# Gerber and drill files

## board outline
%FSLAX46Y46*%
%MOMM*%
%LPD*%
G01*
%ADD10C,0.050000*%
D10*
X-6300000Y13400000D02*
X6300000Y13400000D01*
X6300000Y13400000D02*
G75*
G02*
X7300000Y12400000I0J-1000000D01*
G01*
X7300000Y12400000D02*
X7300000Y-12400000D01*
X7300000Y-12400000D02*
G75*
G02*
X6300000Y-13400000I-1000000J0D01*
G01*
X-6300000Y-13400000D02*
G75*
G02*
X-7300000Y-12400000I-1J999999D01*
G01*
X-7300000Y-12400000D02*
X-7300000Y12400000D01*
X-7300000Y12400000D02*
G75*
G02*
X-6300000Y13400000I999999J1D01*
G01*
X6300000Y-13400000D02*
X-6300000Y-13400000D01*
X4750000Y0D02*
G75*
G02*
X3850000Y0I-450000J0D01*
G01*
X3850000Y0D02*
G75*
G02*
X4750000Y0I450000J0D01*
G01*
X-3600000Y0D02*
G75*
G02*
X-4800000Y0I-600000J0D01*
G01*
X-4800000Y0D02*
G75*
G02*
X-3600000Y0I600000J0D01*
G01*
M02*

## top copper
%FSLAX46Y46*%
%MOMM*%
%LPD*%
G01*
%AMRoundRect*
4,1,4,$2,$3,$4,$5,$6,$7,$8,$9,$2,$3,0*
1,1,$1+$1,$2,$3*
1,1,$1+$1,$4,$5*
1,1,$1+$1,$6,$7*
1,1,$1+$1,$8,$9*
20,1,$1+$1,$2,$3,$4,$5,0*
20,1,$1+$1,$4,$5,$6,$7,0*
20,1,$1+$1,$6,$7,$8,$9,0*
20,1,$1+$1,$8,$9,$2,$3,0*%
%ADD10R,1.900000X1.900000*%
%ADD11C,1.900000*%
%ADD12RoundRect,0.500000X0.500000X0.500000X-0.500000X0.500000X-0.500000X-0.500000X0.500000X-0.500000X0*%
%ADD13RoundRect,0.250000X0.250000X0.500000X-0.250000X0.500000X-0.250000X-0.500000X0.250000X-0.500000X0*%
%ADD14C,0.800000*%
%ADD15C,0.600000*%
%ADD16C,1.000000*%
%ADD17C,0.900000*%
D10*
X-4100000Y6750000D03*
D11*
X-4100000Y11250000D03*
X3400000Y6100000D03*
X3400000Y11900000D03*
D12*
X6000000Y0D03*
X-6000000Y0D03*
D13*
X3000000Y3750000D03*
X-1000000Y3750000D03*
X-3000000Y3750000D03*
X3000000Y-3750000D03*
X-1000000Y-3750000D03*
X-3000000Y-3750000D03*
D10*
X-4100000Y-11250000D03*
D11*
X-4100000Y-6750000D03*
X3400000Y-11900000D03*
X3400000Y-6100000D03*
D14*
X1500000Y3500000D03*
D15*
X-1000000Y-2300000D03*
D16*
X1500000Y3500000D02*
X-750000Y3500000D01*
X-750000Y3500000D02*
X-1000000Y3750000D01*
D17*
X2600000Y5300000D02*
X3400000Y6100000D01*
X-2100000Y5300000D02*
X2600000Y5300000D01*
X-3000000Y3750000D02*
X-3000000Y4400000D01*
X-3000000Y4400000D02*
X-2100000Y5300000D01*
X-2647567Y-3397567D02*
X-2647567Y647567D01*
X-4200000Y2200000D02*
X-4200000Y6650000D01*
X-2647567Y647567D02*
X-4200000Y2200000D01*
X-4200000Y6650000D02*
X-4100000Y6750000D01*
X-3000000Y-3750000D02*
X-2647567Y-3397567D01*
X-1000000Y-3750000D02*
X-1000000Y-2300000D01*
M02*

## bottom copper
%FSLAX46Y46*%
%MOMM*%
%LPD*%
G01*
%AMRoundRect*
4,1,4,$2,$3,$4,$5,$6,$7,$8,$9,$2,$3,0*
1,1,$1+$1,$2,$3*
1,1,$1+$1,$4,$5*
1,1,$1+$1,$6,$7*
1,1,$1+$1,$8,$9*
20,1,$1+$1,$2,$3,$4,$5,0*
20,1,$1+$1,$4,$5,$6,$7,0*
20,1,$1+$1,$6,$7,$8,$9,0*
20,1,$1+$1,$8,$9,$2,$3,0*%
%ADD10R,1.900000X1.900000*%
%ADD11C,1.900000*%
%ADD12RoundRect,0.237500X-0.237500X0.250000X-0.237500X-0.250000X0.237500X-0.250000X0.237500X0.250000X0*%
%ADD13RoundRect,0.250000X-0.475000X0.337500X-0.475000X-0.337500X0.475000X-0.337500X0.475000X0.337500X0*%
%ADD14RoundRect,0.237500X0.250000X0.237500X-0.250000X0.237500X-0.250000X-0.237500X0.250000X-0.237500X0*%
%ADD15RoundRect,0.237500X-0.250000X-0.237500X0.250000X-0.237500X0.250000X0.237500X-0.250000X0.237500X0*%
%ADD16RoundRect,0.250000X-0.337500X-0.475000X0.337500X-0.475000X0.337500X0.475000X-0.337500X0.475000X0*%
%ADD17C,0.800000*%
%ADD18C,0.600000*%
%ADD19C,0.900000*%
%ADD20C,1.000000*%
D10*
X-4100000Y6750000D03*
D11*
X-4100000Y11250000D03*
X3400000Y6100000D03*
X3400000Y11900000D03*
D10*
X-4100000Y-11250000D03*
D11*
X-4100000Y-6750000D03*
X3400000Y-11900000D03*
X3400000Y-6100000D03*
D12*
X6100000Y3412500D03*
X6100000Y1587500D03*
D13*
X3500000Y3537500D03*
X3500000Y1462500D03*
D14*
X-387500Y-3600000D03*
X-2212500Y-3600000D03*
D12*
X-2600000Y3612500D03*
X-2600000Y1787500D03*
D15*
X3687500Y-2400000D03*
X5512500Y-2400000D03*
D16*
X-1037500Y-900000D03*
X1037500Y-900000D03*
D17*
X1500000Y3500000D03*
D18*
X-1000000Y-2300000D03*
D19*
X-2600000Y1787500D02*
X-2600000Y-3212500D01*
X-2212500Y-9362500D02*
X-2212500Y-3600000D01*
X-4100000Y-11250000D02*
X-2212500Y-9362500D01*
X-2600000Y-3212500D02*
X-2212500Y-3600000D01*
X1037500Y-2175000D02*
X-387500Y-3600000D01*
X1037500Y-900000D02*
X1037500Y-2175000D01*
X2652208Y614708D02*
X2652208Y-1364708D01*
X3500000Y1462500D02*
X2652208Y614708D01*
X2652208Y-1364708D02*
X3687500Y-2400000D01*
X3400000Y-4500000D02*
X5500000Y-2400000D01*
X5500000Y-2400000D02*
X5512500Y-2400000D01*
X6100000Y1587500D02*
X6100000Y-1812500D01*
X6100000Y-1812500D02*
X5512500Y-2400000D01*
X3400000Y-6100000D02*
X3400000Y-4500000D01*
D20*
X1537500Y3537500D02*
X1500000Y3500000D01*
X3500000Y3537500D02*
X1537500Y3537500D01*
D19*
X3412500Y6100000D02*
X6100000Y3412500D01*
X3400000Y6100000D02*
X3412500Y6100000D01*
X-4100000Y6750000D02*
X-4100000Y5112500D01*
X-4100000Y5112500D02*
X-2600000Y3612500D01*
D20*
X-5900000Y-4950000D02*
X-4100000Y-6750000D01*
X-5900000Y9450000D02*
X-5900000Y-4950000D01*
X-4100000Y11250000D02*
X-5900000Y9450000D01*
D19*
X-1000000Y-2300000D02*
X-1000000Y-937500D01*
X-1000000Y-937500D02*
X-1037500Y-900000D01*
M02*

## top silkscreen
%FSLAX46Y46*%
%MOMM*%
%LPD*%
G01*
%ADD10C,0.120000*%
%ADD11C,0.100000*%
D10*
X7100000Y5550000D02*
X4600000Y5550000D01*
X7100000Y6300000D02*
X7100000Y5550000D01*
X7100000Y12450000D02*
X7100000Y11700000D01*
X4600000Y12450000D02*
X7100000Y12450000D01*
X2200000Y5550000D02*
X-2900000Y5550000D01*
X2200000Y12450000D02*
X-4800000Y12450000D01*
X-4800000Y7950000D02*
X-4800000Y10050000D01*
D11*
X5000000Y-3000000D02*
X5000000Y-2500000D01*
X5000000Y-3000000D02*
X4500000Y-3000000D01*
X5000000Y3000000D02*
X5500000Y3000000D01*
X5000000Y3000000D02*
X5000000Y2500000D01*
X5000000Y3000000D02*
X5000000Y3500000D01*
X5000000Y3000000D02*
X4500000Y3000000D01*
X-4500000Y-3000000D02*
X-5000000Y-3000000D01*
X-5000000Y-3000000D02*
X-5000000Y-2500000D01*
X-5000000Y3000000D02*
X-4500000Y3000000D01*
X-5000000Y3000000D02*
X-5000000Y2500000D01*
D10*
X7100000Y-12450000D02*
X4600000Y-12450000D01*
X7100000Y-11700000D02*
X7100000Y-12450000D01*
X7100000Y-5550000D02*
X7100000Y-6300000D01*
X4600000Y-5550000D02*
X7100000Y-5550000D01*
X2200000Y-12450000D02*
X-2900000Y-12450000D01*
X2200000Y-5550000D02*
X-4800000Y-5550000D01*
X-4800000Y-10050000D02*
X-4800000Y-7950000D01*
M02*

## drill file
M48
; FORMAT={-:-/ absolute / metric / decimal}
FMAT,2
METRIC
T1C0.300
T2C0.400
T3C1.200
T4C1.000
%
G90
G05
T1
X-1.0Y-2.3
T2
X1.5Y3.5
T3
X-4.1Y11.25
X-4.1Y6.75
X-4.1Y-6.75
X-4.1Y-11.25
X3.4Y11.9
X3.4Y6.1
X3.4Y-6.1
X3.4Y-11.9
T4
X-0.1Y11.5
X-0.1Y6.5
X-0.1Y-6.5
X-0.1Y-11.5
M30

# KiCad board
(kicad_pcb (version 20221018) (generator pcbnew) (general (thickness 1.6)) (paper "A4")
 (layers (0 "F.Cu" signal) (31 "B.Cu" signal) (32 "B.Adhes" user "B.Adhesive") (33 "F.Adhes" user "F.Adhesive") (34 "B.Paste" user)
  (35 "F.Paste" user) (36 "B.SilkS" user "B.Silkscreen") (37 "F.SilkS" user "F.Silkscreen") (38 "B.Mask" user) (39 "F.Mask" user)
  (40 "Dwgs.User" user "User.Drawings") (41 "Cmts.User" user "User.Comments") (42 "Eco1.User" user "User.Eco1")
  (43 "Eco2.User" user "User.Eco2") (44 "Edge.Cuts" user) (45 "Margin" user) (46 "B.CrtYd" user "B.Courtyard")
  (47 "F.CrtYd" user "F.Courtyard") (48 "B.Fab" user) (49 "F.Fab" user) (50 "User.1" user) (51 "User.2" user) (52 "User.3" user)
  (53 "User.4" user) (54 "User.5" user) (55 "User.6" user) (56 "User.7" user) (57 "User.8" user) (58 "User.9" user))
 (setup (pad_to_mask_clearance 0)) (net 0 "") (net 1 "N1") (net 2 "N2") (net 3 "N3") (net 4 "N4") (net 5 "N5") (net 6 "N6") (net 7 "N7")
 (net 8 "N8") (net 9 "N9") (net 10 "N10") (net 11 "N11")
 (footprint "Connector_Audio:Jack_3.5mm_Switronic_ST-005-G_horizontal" (layer "F.Cu") (at 2.4 -9 180)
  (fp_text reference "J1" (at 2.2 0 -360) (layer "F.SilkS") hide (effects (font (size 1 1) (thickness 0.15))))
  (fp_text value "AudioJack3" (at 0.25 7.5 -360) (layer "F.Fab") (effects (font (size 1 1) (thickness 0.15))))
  (fp_line (start -4.7 -3.45) (end -2.2 -3.45) (stroke (width 0.12) (type solid)) (layer "F.SilkS"))
  (fp_line (start -4.7 -2.7) (end -4.7 -3.45) (stroke (width 0.12) (type solid)) (layer "F.SilkS"))
  (fp_line (start -4.7 3.45) (end -4.7 2.7) (stroke (width 0.12) (type solid)) (layer "F.SilkS"))
  (fp_line (start -2.2 3.45) (end -4.7 3.45) (stroke (width 0.12) (type solid)) (layer "F.SilkS"))
  (fp_line (start 0.2 -3.45) (end 5.3 -3.45) (stroke (width 0.12) (type solid)) (layer "F.SilkS"))
  (fp_line (start 0.2 3.45) (end 7.2 3.45) (stroke (width 0.12) (type solid)) (layer "F.SilkS"))
  (fp_line (start 7.2 -1.05) (end 7.2 1.05) (stroke (width 0.12) (type solid)) (layer "F.SilkS"))
  (pad "" np_thru_hole circle (at 2.5 -2.5 180) (size 1 1) (drill 1) (layers "*.Cu" "*.Mask"))
  (pad "" np_thru_hole circle (at 2.5 2.5 180) (size 1 1) (drill 1) (layers "*.Cu" "*.Mask"))
  (pad "R" thru_hole rect (at 6.5 -2.25 180) (size 1.9 1.9) (drill 1.2) (layers "*.Cu" "*.Mask") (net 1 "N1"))
  (pad "S" thru_hole circle (at 6.5 2.25 180) (size 1.9 1.9) (drill 1.2) (layers "*.Cu" "*.Mask") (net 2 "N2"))
  (pad "T" thru_hole circle (at -1 -2.9 180) (size 1.9 1.9) (drill 1.2) (layers "*.Cu" "*.Mask") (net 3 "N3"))
  (pad "T" thru_hole circle (at -1 2.9 180) (size 1.9 1.9) (drill 1.2) (layers "*.Cu" "*.Mask") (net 3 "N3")))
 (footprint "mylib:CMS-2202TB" (layer "F.Cu") (at 0 0 180)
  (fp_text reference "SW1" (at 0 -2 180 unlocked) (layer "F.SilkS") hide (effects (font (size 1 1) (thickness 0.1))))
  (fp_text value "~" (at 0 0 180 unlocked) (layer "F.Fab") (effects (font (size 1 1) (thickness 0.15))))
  (fp_line (start -5 -3) (end -5 -2.5) (stroke (width 0.1) (type default)) (layer "F.SilkS"))
  (fp_line (start -5 -3) (end -4.5 -3) (stroke (width 0.1) (type default)) (layer "F.SilkS"))
  (fp_line (start -5 3) (end -5.5 3) (stroke (width 0.1) (type default)) (layer "F.SilkS"))
  (fp_line (start -5 3) (end -5 2.5) (stroke (width 0.1) (type default)) (layer "F.SilkS"))
  (fp_line (start -5 3) (end -5 3.5) (stroke (width 0.1) (type default)) (layer "F.SilkS"))
  (fp_line (start -5 3) (end -4.5 3) (stroke (width 0.1) (type default)) (layer "F.SilkS"))
  (fp_line (start 4.5 -3) (end 5 -3) (stroke (width 0.1) (type default)) (layer "F.SilkS"))
  (fp_line (start 5 -3) (end 5 -2.5) (stroke (width 0.1) (type default)) (layer "F.SilkS"))
  (fp_line (start 5 3) (end 4.5 3) (stroke (width 0.1) (type default)) (layer "F.SilkS"))
  (fp_line (start 5 3) (end 5 2.5) (stroke (width 0.1) (type default)) (layer "F.SilkS"))
  (fp_circle (center -4.3 0) (end -3.85 0) (stroke (width 0.05) (type default)) (fill none) (layer "Edge.Cuts"))
  (fp_circle (center 4.2 0) (end 4.8 0) (stroke (width 0.05) (type default)) (fill none) (layer "Edge.Cuts"))
  (pad "" smd roundrect (at -6 0 180) (size 2 2) (layers "F.Cu" "F.Paste" "F.Mask") (roundrect_rratio 0.25) (thermal_bridge_angle 45))
  (pad "" smd roundrect (at 6 0 180) (size 2 2) (layers "F.Cu" "F.Paste" "F.Mask") (roundrect_rratio 0.25) (thermal_bridge_angle 45))
  (pad "1" smd roundrect (at -3 3.75 180) (size 1 1.5) (layers "F.Cu" "F.Paste" "F.Mask") (roundrect_rratio 0.25) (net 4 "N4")
   (thermal_bridge_angle 45))
  (pad "2" smd roundrect (at 1 3.75 180) (size 1 1.5) (layers "F.Cu" "F.Paste" "F.Mask") (roundrect_rratio 0.25) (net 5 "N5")
   (thermal_bridge_angle 45))
  (pad "3" smd roundrect (at 3 3.75 180) (size 1 1.5) (layers "F.Cu" "F.Paste" "F.Mask") (roundrect_rratio 0.25) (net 3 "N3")
   (thermal_bridge_angle 45))
  (pad "4" smd roundrect (at -3 -3.75 180) (size 1 1.5) (layers "F.Cu" "F.Paste" "F.Mask") (roundrect_rratio 0.25) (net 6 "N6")
   (thermal_bridge_angle 45))
  (pad "5" smd roundrect (at 1 -3.75 180) (size 1 1.5) (layers "F.Cu" "F.Paste" "F.Mask") (roundrect_rratio 0.25) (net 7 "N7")
   (thermal_bridge_angle 45))
  (pad "6" smd roundrect (at 3 -3.75 180) (size 1 1.5) (layers "F.Cu" "F.Paste" "F.Mask") (roundrect_rratio 0.25) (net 1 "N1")
   (thermal_bridge_angle 45)))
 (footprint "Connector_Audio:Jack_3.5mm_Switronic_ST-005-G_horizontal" (layer "F.Cu") (at 2.4 9 180)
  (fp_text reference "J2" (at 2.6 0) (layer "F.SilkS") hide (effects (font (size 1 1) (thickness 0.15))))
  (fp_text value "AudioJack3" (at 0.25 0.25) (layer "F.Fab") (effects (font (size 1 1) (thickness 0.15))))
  (fp_line (start -4.7 -3.45) (end -2.2 -3.45) (stroke (width 0.12) (type solid)) (layer "F.SilkS"))
  (fp_line (start -4.7 -2.7) (end -4.7 -3.45) (stroke (width 0.12) (type solid)) (layer "F.SilkS"))
  (fp_line (start -4.7 3.45) (end -4.7 2.7) (stroke (width 0.12) (type solid)) (layer "F.SilkS"))
  (fp_line (start -2.2 3.45) (end -4.7 3.45) (stroke (width 0.12) (type solid)) (layer "F.SilkS"))
  (fp_line (start 0.2 -3.45) (end 5.3 -3.45) (stroke (width 0.12) (type solid)) (layer "F.SilkS"))
  (fp_line (start 0.2 3.45) (end 7.2 3.45) (stroke (width 0.12) (type solid)) (layer "F.SilkS"))
  (fp_line (start 7.2 -1.05) (end 7.2 1.05) (stroke (width 0.12) (type solid)) (layer "F.SilkS"))
  (pad "" np_thru_hole circle (at 2.5 -2.5 180) (size 1 1) (drill 1) (layers "*.Cu" "*.Mask"))
  (pad "" np_thru_hole circle (at 2.5 2.5 180) (size 1 1) (drill 1) (layers "*.Cu" "*.Mask"))
  (pad "R" thru_hole rect (at 6.5 -2.25 180) (size 1.9 1.9) (drill 1.2) (layers "*.Cu" "*.Mask") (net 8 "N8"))
  (pad "S" thru_hole circle (at 6.5 2.25 180) (size 1.9 1.9) (drill 1.2) (layers "*.Cu" "*.Mask") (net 2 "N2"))
  (pad "T" thru_hole circle (at -1 -2.9 180) (size 1.9 1.9) (drill 1.2) (layers "*.Cu" "*.Mask") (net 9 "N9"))
  (pad "T" thru_hole circle (at -1 2.9 180) (size 1.9 1.9) (drill 1.2) (layers "*.Cu" "*.Mask") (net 9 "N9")))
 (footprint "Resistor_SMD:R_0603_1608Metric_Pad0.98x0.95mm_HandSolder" (layer "B.Cu") (at 6.1 -2.5 -90)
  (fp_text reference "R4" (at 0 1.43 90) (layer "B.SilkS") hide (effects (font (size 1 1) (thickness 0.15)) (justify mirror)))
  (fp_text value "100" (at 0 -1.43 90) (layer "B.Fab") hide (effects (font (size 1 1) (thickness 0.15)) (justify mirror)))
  (pad "1" smd roundrect (at -0.9125 0 270) (size 0.975 0.95) (layers "B.Cu" "B.Paste" "B.Mask") (roundrect_rratio 0.25) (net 3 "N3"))
  (pad "2" smd roundrect (at 0.9125 0 270) (size 0.975 0.95) (layers "B.Cu" "B.Paste" "B.Mask") (roundrect_rratio 0.25) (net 9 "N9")))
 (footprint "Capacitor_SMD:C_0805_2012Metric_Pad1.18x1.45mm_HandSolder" (layer "B.Cu") (at 3.5 -2.5 -90)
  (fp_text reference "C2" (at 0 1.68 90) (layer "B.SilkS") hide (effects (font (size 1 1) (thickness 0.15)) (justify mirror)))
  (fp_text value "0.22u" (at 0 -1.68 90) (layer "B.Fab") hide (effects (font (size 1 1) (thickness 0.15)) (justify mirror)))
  (pad "1" smd roundrect (at -1.0375 0 270) (size 1.175 1.45) (layers "B.Cu" "B.Paste" "B.Mask") (roundrect_rratio 0.2127659574)
   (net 5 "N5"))
  (pad "2" smd roundrect (at 1.0375 0 270) (size 1.175 1.45) (layers "B.Cu" "B.Paste" "B.Mask") (roundrect_rratio 0.2127659574)
   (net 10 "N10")))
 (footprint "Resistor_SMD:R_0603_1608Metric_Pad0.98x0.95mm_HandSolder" (layer "B.Cu") (at -1.3 3.6 180)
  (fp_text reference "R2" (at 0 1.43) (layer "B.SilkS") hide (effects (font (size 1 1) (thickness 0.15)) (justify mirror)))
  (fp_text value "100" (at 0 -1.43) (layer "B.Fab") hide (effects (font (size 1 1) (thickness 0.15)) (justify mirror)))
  (pad "1" smd roundrect (at -0.9125 0 180) (size 0.975 0.95) (layers "B.Cu" "B.Paste" "B.Mask") (roundrect_rratio 0.25) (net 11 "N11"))
  (pad "2" smd roundrect (at 0.9125 0 180) (size 0.975 0.95) (layers "B.Cu" "B.Paste" "B.Mask") (roundrect_rratio 0.25) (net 8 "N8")))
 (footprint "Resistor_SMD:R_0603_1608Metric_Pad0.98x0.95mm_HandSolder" (layer "B.Cu") (at -2.6 -2.7 -90)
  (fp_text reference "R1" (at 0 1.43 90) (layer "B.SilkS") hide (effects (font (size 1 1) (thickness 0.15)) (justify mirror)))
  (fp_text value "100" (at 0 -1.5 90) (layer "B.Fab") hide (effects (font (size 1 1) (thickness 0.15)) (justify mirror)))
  (pad "1" smd roundrect (at -0.9125 0 270) (size 0.975 0.95) (layers "B.Cu" "B.Paste" "B.Mask") (roundrect_rratio 0.25) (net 1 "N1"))
  (pad "2" smd roundrect (at 0.9125 0 270) (size 0.975 0.95) (layers "B.Cu" "B.Paste" "B.Mask") (roundrect_rratio 0.25) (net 8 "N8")))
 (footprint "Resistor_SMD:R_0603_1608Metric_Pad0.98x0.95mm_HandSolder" (layer "B.Cu") (at 4.6 2.4)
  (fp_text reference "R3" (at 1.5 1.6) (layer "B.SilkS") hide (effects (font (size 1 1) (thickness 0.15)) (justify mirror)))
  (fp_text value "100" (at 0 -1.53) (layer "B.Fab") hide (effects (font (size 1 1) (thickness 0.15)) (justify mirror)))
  (pad "1" smd roundrect (at -0.9125 0) (size 0.975 0.95) (layers "B.Cu" "B.Paste" "B.Mask") (roundrect_rratio 0.25) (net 10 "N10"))
  (pad "2" smd roundrect (at 0.9125 0) (size 0.975 0.95) (layers "B.Cu" "B.Paste" "B.Mask") (roundrect_rratio 0.25) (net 9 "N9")))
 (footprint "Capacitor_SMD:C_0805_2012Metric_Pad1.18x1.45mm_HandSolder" (layer "B.Cu") (at 0 0.9)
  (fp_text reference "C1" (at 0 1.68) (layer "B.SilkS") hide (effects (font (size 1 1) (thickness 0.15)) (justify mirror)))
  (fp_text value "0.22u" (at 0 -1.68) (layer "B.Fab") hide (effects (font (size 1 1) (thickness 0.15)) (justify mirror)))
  (pad "1" smd roundrect (at -1.0375 0) (size 1.175 1.45) (layers "B.Cu" "B.Paste" "B.Mask") (roundrect_rratio 0.2127659574) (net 7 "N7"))
  (pad "2" smd roundrect (at 1.0375 0) (size 1.175 1.45) (layers "B.Cu" "B.Paste" "B.Mask") (roundrect_rratio 0.2127659574) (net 11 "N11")))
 (gr_line (start -6.3 -13.4) (end 6.3 -13.4) (stroke (width 0.05) (type default)) (layer "Edge.Cuts"))
 (gr_arc (start 6.3 -13.4) (mid 7.007107 -13.107107) (end 7.3 -12.4) (stroke (width 0.05) (type default)) (layer "Edge.Cuts"))
 (gr_line (start 7.3 -12.4) (end 7.3 12.4) (stroke (width 0.05) (type default)) (layer "Edge.Cuts"))
 (gr_arc (start 7.3 12.4) (mid 7.007107 13.107107) (end 6.3 13.4) (stroke (width 0.05) (type default)) (layer "Edge.Cuts"))
 (gr_arc (start -6.3 13.4) (mid -7.007107 13.107107) (end -7.3 12.4) (stroke (width 0.05) (type default)) (layer "Edge.Cuts"))
 (gr_line (start -7.3 12.4) (end -7.3 -12.4) (stroke (width 0.05) (type default)) (layer "Edge.Cuts"))
 (gr_arc (start -7.3 -12.4) (mid -7.007107 -13.107107) (end -6.3 -13.4) (stroke (width 0.05) (type default)) (layer "Edge.Cuts"))
 (gr_line (start 6.3 13.4) (end -6.3 13.4) (stroke (width 0.05) (type default)) (layer "Edge.Cuts"))
 (segment (start -2.6 -1.7875) (end -2.6 3.2125) (width 0.9) (layer "B.Cu") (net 8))
 (segment (start -2.2125 9.3625) (end -2.2125 3.6) (width 0.9) (layer "B.Cu") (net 8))
 (segment (start -4.1 11.25) (end -2.2125 9.3625) (width 0.9) (layer "B.Cu") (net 8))
 (segment (start -2.6 3.2125) (end -2.2125 3.6) (width 0.9) (layer "B.Cu") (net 8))
 (segment (start 1.0375 2.175) (end -0.3875 3.6) (width 0.9) (layer "B.Cu") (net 11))
 (segment (start 1.0375 0.9) (end 1.0375 2.175) (width 0.9) (layer "B.Cu") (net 11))
 (segment (start 2.652208 -0.614708) (end 2.652208 1.364708) (width 0.9) (layer "B.Cu") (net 10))
 (segment (start 3.5 -1.4625) (end 2.652208 -0.614708) (width 0.9) (layer "B.Cu") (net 10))
 (segment (start 2.652208 1.364708) (end 3.6875 2.4) (width 0.9) (layer "B.Cu") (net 10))
 (segment (start 3.4 4.5) (end 5.5 2.4) (width 0.9) (layer "B.Cu") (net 9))
 (segment (start 5.5 2.4) (end 5.5125 2.4) (width 0.9) (layer "B.Cu") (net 9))
 (segment (start 6.1 -1.5875) (end 6.1 1.8125) (width 0.9) (layer "B.Cu") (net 9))
 (segment (start 6.1 1.8125) (end 5.5125 2.4) (width 0.9) (layer "B.Cu") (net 9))
 (segment (start 3.4 6.1) (end 3.4 4.5) (width 0.9) (layer "B.Cu") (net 9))
 (segment (start 1.5 -3.5) (end -0.75 -3.5) (width 1) (layer "F.Cu") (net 5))
 (segment (start -0.75 -3.5) (end -1 -3.75) (width 1) (layer "F.Cu") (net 5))
 (via (at 1.5 -3.5) (size 0.8) (drill 0.4) (layers "F.Cu" "B.Cu") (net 5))
 (segment (start 1.5375 -3.5375) (end 1.5 -3.5) (width 1) (layer "B.Cu") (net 5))
 (segment (start 3.5 -3.5375) (end 1.5375 -3.5375) (width 1) (layer "B.Cu") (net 5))
 (segment (start 2.6 -5.3) (end 3.4 -6.1) (width 0.9) (layer "F.Cu") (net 3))
 (segment (start -2.1 -5.3) (end 2.6 -5.3) (width 0.9) (layer "F.Cu") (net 3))
 (segment (start -3 -3.75) (end -3 -4.4) (width 0.9) (layer "F.Cu") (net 3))
 (segment (start -3 -4.4) (end -2.1 -5.3) (width 0.9) (layer "F.Cu") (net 3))
 (segment (start 3.4125 -6.1) (end 6.1 -3.4125) (width 0.9) (layer "B.Cu") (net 3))
 (segment (start 3.4 -6.1) (end 3.4125 -6.1) (width 0.9) (layer "B.Cu") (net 3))
 (segment (start -2.647567 3.397567) (end -2.647567 -0.647567) (width 0.9) (layer "F.Cu") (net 1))
 (segment (start -4.2 -2.2) (end -4.2 -6.65) (width 0.9) (layer "F.Cu") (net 1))
 (segment (start -2.647567 -0.647567) (end -4.2 -2.2) (width 0.9) (layer "F.Cu") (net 1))
 (segment (start -4.2 -6.65) (end -4.1 -6.75) (width 0.9) (layer "F.Cu") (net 1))
 (segment (start -3 3.75) (end -2.647567 3.397567) (width 0.9) (layer "F.Cu") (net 1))
 (segment (start -4.1 -6.75) (end -4.1 -5.1125) (width 0.9) (layer "B.Cu") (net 1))
 (segment (start -4.1 -5.1125) (end -2.6 -3.6125) (width 0.9) (layer "B.Cu") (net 1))
 (segment (start -5.9 4.95) (end -4.1 6.75) (width 1) (layer "B.Cu") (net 2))
 (segment (start -5.9 -9.45) (end -5.9 4.95) (width 1) (layer "B.Cu") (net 2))
 (segment (start -4.1 -11.25) (end -5.9 -9.45) (width 1) (layer "B.Cu") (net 2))
 (segment (start -1 3.75) (end -1 2.3) (width 0.9) (layer "F.Cu") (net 7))
 (via (at -1 2.3) (size 0.6) (drill 0.3) (layers "F.Cu" "B.Cu") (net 7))
 (segment (start -1 2.3) (end -1 0.9375) (width 0.9) (layer "B.Cu") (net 7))
 (segment (start -1 0.9375) (end -1.0375 0.9) (width 0.9) (layer "B.Cu") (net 7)))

